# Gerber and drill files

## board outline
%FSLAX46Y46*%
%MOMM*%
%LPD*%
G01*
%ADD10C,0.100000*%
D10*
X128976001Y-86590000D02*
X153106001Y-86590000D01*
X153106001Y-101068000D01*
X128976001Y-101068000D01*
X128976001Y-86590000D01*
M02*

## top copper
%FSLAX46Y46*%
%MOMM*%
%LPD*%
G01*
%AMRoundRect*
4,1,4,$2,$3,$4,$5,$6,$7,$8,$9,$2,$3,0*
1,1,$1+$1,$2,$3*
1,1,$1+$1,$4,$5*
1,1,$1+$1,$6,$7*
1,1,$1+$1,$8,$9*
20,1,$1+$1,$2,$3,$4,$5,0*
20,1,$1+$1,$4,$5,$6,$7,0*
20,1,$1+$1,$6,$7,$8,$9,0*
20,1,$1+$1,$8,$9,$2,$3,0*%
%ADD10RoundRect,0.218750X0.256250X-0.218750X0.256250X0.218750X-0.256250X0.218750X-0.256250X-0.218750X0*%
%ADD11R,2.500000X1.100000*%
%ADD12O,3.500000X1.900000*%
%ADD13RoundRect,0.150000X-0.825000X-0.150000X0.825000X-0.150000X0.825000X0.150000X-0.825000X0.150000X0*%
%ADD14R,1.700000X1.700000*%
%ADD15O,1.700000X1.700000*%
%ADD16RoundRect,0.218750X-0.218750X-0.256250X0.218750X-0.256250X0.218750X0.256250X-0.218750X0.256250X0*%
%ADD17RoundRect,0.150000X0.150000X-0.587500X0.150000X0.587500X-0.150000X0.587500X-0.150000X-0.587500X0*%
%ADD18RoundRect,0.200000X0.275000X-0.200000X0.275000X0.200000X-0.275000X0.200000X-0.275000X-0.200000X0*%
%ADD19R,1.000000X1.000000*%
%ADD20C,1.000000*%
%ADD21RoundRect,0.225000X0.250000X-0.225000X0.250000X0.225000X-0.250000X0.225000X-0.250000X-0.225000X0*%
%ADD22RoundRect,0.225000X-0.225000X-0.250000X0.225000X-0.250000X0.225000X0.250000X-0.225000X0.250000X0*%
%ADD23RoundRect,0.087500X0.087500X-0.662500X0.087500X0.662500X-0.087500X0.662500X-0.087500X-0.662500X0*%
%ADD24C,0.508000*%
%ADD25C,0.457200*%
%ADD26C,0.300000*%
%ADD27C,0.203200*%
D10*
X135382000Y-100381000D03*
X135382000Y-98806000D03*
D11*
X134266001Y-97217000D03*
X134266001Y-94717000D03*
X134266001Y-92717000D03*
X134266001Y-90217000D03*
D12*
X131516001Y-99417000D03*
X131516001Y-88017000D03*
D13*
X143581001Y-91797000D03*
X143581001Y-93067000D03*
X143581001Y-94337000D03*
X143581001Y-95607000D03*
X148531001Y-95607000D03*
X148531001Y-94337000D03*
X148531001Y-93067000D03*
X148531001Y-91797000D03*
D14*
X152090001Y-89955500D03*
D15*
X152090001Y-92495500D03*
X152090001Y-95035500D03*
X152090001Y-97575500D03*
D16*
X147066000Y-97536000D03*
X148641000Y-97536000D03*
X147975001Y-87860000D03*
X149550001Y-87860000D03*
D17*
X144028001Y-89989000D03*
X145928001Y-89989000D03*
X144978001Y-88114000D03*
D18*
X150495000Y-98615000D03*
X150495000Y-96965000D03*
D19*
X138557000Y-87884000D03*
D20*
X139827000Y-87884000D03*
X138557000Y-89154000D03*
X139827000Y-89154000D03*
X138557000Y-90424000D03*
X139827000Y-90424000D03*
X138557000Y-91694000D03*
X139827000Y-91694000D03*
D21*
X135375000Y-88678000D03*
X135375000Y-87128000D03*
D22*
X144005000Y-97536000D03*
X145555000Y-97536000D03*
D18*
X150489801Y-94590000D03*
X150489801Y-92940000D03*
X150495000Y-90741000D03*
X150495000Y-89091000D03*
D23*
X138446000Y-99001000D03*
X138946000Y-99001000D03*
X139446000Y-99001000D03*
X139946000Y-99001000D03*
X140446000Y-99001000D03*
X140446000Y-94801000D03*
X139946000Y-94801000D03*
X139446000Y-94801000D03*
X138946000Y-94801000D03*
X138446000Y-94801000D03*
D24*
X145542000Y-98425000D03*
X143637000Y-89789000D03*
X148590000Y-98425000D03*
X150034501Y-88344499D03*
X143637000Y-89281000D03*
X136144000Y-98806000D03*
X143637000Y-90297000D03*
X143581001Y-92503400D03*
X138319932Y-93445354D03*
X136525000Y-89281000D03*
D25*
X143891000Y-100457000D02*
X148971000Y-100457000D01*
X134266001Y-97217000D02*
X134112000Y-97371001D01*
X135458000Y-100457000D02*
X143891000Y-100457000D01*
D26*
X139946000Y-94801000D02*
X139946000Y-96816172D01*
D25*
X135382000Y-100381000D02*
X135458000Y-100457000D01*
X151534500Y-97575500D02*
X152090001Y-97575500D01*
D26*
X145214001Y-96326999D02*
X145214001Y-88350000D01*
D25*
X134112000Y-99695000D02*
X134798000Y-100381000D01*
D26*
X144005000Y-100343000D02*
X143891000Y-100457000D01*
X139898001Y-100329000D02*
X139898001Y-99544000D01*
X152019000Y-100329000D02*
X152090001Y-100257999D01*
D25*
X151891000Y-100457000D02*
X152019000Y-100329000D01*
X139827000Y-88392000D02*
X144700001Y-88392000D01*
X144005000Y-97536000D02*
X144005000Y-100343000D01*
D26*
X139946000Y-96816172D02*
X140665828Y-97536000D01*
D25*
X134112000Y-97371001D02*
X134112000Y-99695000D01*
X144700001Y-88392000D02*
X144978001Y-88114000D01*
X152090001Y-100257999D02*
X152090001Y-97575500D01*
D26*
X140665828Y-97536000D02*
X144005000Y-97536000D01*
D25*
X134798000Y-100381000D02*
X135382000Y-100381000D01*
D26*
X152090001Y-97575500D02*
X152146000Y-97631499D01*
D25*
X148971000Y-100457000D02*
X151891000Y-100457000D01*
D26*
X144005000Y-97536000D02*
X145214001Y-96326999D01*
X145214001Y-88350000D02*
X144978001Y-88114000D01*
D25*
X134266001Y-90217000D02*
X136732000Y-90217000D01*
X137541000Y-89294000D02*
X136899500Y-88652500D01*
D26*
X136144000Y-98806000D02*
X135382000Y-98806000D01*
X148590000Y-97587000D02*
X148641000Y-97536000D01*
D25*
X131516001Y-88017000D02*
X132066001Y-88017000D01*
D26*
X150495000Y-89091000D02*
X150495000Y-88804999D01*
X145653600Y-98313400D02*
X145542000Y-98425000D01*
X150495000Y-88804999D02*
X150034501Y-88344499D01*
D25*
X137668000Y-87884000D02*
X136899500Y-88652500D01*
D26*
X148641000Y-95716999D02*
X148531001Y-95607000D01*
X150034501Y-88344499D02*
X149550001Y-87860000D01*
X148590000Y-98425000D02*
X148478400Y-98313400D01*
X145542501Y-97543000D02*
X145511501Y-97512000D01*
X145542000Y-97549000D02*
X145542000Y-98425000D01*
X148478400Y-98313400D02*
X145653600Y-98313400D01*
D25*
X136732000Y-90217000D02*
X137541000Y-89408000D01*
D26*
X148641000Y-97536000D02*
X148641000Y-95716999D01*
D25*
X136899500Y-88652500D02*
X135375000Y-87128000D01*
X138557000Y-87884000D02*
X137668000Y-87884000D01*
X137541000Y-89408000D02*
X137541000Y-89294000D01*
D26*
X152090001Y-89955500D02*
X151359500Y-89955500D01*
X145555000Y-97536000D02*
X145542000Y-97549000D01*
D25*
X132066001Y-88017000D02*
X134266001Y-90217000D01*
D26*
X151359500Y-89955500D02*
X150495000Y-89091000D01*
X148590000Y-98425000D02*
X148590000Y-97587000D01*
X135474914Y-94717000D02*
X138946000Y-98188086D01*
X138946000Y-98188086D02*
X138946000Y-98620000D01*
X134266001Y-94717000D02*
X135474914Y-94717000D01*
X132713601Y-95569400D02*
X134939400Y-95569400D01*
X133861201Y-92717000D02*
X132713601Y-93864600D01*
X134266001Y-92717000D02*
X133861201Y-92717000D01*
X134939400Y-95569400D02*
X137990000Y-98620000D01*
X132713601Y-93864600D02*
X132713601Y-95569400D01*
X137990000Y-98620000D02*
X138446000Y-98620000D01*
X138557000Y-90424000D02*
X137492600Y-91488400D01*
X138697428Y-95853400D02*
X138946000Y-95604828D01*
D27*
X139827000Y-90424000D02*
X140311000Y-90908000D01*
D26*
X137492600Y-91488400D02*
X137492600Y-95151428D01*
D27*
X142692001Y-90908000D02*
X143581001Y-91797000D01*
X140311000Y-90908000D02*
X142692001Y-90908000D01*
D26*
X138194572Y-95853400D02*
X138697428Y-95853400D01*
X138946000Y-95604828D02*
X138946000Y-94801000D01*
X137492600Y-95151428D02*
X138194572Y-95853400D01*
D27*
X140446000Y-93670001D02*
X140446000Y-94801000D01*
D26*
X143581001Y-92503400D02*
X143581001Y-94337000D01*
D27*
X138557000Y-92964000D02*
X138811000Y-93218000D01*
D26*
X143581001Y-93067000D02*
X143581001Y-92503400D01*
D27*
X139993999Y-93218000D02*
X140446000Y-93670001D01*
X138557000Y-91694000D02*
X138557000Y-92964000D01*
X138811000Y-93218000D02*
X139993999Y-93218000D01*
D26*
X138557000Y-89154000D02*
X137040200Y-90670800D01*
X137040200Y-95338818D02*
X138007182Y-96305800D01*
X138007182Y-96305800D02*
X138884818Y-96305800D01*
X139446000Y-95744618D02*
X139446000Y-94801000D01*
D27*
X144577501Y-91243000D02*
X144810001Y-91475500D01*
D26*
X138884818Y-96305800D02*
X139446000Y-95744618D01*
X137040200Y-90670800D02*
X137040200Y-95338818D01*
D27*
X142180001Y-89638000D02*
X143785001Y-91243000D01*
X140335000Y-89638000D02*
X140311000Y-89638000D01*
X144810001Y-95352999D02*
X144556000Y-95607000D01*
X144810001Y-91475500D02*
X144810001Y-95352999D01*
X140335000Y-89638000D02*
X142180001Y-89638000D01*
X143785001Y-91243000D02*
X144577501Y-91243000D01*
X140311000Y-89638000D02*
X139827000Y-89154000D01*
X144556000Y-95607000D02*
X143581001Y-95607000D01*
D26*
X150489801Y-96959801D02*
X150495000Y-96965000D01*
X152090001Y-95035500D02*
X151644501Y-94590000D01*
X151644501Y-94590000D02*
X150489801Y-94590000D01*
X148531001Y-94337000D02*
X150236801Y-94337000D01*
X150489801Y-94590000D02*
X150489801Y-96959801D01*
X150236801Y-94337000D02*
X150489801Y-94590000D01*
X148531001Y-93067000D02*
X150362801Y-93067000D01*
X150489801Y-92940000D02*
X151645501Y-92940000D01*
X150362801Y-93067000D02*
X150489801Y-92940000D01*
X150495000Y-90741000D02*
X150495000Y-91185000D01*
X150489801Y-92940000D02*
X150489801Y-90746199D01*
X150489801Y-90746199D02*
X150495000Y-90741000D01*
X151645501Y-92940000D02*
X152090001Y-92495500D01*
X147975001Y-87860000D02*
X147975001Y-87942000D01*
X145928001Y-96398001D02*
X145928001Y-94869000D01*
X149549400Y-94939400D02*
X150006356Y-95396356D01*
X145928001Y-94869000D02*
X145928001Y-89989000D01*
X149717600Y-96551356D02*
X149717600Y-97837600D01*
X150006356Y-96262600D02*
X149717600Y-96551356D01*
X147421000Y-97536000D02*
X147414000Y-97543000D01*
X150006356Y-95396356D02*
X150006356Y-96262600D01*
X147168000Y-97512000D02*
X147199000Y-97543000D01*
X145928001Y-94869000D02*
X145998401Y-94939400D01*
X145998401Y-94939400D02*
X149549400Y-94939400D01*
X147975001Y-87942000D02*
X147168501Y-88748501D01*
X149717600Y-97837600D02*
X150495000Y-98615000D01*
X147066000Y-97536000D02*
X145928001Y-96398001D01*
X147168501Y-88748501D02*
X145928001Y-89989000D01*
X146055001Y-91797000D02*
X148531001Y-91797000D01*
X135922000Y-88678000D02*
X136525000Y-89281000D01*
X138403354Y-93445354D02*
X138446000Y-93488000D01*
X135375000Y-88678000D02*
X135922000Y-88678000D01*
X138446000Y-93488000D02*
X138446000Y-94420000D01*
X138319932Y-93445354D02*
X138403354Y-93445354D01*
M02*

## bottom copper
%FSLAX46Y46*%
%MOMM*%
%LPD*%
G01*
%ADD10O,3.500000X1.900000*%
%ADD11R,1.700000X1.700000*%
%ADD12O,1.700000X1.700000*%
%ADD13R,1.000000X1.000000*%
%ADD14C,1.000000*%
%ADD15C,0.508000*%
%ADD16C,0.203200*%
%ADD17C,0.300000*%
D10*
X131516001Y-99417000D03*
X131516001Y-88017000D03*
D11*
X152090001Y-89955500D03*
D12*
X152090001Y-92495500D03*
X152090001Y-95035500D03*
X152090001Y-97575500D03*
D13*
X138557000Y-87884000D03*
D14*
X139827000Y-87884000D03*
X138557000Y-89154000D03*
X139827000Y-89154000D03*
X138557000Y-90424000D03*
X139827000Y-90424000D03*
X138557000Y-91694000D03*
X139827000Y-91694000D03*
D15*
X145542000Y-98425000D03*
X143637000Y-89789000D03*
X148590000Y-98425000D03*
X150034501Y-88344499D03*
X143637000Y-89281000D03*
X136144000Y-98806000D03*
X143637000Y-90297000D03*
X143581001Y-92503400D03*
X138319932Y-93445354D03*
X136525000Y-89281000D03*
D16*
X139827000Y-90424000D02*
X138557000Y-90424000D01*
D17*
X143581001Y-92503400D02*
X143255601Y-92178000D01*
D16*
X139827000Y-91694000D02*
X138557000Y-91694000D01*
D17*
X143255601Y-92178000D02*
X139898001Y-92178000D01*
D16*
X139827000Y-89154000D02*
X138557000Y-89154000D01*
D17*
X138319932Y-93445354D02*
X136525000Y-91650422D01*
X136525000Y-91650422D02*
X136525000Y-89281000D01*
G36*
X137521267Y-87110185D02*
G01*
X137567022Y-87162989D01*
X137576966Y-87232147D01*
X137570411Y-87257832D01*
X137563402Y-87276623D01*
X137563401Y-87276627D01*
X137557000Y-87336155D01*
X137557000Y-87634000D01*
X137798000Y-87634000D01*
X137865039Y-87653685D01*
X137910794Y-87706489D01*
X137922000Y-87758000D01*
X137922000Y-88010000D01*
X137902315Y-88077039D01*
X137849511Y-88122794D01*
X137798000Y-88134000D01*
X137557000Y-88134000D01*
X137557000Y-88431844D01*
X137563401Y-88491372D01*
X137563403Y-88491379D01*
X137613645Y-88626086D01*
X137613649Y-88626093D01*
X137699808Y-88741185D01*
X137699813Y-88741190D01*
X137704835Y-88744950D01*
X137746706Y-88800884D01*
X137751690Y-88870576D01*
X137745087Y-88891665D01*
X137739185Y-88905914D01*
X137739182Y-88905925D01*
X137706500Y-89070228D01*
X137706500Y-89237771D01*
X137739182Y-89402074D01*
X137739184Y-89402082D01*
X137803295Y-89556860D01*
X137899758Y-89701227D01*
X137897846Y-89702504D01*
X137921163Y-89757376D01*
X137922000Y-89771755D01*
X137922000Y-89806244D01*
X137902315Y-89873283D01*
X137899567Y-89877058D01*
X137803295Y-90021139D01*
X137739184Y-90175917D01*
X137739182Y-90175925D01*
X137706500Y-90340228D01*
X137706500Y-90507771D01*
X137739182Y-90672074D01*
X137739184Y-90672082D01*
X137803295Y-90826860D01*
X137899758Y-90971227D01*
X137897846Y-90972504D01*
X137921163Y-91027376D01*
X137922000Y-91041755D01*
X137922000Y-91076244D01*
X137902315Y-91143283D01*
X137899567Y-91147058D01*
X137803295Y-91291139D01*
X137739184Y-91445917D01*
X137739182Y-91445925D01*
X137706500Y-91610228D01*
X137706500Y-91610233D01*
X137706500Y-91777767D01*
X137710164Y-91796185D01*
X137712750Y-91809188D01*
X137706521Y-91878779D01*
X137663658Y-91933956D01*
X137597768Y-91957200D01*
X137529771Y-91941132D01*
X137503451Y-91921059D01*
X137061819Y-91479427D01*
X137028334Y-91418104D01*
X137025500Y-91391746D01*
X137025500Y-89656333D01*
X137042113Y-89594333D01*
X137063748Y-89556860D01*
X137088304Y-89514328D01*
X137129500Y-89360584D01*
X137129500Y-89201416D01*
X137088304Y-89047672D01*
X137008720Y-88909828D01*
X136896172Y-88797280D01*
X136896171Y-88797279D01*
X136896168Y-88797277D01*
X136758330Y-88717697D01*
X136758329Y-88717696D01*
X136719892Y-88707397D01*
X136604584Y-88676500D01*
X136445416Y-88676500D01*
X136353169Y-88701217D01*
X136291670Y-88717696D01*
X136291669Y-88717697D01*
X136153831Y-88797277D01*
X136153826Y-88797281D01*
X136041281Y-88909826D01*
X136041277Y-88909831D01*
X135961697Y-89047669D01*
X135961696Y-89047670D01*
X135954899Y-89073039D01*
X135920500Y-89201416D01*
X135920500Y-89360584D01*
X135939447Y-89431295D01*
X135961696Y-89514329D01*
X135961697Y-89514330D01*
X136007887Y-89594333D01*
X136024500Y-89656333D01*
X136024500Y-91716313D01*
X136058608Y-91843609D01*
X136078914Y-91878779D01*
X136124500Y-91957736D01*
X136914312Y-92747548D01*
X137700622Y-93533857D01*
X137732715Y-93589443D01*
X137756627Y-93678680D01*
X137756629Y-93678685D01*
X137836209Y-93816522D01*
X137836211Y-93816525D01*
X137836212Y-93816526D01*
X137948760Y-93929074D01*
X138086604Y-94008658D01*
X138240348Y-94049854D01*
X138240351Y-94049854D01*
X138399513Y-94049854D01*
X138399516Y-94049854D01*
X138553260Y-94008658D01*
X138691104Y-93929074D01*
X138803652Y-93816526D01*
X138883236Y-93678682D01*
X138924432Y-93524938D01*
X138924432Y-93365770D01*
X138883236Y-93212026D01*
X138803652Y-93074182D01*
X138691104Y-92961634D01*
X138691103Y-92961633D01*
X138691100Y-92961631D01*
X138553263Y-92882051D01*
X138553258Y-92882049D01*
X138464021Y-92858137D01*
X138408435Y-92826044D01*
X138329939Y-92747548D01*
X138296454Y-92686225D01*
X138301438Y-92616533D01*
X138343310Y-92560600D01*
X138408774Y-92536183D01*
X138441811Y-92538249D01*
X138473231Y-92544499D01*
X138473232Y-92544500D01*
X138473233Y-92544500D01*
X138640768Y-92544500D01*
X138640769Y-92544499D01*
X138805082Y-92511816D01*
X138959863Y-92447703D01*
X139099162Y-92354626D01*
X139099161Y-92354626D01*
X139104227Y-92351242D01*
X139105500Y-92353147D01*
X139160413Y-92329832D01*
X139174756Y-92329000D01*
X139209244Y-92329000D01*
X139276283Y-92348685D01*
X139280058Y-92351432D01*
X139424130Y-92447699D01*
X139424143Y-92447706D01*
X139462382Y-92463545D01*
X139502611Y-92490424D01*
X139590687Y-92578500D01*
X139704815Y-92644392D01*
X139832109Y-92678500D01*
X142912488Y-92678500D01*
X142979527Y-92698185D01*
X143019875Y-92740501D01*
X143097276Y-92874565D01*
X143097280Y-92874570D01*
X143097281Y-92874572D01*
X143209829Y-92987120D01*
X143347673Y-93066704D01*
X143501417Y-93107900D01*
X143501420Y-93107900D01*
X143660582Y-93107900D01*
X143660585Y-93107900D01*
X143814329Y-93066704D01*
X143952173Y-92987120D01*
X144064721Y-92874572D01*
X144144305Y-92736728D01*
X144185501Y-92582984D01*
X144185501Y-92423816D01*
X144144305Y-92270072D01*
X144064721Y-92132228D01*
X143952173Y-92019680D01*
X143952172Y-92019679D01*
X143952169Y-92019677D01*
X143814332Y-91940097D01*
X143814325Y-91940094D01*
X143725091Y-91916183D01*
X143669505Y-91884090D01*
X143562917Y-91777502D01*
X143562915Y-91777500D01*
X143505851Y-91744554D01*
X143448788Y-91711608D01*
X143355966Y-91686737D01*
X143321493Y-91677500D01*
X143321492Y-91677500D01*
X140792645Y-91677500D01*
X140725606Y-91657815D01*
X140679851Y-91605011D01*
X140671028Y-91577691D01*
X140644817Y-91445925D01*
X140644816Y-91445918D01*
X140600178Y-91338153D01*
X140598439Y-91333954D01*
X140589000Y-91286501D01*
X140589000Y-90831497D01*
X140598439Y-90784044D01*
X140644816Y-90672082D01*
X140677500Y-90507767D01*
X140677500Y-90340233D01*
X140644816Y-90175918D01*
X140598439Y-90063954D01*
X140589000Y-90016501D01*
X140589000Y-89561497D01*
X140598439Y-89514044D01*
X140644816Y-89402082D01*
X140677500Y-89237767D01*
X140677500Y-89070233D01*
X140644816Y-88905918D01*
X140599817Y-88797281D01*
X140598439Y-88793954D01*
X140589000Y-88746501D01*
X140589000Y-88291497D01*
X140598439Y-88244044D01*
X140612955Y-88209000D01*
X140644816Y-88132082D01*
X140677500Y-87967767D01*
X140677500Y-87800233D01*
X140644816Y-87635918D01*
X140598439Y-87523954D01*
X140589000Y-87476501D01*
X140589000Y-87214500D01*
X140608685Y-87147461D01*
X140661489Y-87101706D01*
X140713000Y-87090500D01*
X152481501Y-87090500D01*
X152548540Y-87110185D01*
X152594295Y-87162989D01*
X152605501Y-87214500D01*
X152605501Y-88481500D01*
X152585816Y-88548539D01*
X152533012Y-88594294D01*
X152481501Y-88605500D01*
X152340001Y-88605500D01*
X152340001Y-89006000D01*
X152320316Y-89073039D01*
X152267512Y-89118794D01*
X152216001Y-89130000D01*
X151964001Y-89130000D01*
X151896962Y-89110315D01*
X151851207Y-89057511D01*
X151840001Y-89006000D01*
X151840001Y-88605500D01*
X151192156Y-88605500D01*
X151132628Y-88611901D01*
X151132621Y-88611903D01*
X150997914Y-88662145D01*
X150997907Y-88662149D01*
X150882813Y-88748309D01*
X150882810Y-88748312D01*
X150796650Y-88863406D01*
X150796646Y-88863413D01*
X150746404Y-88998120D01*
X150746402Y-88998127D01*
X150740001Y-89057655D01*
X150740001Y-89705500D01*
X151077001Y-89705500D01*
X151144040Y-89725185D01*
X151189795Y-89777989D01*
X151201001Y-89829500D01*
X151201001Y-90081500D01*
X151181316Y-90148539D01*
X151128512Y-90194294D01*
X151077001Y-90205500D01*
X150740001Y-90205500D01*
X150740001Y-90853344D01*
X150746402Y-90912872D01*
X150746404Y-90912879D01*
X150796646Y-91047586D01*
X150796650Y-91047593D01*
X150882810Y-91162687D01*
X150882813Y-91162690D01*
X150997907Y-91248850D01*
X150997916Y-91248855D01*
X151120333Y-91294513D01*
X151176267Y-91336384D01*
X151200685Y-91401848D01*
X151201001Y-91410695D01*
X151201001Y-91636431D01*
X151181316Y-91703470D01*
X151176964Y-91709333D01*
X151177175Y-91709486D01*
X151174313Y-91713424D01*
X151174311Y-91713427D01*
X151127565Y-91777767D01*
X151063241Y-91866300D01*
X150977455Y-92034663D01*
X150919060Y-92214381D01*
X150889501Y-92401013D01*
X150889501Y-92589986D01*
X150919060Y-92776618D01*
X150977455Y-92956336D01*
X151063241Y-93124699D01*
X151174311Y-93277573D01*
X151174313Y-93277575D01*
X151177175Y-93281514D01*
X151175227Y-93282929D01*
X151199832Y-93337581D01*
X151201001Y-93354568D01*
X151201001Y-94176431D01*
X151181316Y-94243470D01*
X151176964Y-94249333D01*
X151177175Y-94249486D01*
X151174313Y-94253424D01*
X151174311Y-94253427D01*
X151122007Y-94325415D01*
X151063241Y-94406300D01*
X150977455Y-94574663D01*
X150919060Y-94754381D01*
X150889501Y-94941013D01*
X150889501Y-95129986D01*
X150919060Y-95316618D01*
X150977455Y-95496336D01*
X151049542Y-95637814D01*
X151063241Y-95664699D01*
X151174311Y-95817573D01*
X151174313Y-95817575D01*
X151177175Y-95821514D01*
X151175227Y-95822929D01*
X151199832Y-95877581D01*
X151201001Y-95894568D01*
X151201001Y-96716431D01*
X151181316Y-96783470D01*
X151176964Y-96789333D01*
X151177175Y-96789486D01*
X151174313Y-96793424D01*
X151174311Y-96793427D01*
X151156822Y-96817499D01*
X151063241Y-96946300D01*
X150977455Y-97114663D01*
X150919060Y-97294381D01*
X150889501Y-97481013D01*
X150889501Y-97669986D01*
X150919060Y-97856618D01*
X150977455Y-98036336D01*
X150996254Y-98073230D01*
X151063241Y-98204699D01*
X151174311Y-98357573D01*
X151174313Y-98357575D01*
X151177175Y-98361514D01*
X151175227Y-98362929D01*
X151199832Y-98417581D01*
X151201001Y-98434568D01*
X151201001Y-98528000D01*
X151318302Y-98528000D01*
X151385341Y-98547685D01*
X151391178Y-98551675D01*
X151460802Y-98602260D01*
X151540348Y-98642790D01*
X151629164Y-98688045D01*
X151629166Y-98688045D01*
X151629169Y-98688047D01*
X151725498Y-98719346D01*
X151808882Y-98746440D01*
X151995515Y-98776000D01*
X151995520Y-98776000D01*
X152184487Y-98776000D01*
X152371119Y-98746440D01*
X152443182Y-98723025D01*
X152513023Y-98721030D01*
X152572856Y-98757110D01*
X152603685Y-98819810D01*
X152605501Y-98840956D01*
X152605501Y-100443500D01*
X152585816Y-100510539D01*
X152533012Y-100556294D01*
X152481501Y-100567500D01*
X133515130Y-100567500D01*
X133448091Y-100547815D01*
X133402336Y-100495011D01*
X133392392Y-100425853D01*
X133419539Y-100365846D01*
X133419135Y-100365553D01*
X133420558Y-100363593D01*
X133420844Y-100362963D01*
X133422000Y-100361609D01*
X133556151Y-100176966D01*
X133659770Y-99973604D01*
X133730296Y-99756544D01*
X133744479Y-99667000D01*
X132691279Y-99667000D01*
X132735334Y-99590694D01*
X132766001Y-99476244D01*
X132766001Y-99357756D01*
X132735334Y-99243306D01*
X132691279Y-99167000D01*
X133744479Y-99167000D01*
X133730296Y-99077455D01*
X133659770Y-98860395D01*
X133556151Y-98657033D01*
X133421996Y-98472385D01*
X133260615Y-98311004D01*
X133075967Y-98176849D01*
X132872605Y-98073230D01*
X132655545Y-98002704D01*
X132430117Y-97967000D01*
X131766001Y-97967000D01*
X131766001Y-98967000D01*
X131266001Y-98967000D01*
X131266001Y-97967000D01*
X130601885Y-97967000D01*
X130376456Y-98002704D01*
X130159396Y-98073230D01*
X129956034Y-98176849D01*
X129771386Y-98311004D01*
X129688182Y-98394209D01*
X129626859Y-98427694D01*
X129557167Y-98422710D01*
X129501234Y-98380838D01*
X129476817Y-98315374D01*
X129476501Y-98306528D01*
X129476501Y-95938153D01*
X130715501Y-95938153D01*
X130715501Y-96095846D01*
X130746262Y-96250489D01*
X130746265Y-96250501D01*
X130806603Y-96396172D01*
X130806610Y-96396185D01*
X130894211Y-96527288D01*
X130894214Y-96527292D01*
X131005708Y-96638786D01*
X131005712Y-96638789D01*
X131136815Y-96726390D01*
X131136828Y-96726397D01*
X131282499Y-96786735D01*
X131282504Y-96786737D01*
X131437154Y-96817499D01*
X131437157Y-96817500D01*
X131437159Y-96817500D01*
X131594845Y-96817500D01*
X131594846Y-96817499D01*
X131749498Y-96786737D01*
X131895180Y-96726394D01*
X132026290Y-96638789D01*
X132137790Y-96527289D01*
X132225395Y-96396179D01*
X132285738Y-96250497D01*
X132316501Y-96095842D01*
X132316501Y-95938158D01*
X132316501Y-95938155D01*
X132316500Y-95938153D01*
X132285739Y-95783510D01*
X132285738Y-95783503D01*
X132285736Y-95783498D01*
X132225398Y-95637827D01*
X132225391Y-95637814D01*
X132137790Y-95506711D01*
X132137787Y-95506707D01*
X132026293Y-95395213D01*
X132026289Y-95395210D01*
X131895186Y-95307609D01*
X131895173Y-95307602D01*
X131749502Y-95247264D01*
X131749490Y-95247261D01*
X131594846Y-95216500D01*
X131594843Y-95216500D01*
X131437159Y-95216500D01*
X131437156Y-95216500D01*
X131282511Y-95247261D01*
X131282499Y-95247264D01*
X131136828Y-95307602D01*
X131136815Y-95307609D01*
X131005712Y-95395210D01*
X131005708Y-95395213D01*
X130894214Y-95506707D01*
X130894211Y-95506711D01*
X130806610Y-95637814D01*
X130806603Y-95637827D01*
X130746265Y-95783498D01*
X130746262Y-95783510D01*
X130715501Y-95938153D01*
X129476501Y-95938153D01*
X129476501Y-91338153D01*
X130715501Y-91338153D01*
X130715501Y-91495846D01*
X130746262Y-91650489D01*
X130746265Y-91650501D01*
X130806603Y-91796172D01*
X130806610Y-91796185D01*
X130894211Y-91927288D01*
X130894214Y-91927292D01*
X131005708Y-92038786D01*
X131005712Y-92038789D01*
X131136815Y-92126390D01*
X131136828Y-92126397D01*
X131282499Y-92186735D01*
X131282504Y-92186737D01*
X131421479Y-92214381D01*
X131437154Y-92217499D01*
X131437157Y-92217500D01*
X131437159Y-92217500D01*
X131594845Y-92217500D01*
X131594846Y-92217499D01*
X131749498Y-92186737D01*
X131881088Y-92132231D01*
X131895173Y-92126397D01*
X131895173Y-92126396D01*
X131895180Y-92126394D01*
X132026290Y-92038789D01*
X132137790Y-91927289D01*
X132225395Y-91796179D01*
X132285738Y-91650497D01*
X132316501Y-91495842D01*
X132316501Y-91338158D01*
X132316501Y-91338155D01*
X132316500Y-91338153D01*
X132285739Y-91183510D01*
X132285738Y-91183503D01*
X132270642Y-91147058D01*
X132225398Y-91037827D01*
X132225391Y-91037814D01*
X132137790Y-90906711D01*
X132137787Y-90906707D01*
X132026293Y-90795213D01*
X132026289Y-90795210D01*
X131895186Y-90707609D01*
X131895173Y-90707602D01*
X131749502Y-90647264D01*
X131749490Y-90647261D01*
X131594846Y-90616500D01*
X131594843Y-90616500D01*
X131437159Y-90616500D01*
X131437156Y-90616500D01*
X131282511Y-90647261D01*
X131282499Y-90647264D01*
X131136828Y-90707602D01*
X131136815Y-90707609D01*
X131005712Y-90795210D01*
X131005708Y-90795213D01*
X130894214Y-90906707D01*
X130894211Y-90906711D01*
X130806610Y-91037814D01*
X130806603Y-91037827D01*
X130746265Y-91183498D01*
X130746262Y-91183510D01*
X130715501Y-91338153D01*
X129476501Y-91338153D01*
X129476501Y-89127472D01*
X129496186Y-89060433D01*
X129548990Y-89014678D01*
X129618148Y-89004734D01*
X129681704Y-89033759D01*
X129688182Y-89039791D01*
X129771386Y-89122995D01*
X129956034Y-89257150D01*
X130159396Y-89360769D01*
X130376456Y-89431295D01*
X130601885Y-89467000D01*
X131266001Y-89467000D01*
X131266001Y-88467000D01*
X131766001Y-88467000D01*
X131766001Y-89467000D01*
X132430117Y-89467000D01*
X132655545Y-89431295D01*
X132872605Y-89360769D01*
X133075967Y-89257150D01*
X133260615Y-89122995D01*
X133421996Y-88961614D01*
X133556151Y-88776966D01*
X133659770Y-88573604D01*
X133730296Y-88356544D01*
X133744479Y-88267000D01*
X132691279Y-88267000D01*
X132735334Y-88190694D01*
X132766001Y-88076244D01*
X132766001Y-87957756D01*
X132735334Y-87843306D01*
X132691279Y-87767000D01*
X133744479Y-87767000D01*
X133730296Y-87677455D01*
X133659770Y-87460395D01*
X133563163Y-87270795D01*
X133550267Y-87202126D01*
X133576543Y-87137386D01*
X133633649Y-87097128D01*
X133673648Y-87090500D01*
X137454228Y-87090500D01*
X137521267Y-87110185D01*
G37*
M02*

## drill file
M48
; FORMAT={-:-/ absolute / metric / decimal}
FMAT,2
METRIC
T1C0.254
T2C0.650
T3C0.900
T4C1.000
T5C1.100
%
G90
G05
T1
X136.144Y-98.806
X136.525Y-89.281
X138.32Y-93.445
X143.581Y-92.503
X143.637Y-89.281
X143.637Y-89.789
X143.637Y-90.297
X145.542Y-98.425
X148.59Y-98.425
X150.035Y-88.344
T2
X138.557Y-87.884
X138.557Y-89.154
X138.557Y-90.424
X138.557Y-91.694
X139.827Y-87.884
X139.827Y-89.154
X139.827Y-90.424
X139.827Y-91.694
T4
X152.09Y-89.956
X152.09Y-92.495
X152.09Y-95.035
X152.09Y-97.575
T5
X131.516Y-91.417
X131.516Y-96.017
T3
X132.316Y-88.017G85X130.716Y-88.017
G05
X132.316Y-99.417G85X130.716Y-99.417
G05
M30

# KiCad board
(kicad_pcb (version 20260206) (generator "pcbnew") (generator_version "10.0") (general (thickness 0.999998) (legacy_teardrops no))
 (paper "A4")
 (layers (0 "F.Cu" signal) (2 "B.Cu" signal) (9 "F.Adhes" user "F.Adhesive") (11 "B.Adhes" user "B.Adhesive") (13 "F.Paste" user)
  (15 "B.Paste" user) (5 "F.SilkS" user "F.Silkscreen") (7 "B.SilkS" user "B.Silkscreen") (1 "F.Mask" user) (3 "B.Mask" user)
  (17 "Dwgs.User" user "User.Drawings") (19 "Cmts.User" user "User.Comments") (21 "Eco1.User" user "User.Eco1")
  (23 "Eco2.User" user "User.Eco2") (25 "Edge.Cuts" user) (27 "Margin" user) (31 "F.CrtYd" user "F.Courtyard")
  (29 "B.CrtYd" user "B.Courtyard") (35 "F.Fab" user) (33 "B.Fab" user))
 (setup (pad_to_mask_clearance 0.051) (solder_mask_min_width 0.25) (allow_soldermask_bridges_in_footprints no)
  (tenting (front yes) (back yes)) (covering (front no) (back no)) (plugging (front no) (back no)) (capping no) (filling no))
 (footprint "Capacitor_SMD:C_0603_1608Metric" (layer "F.Cu") (at 135.382 99.5935 90)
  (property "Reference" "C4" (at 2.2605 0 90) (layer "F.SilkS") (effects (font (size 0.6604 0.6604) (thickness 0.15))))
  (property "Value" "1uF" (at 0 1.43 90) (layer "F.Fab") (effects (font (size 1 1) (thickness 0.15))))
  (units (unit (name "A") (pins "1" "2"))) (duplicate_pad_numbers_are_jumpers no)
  (pad "1" smd roundrect (at -0.7875 0 90) (size 0.875 0.95) (layers "F.Cu" "F.Mask" "F.Paste") (roundrect_rratio 0.25) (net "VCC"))
  (pad "2" smd roundrect (at 0.7875 0 90) (size 0.875 0.95) (layers "F.Cu" "F.Mask" "F.Paste") (roundrect_rratio 0.25) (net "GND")))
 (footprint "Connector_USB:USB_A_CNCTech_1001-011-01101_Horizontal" (layer "F.Cu") (at 124.616001 93.717 180)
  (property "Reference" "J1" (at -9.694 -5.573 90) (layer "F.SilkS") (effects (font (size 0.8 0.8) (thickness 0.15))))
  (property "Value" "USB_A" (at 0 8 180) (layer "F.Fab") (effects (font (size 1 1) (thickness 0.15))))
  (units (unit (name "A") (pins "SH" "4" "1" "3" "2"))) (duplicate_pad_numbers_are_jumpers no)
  (pad "" np_thru_hole circle (at -6.9 -2.3 180) (size 1.1 1.1) (drill 1.1) (layers "*.Cu" "*.Mask"))
  (pad "" np_thru_hole circle (at -6.9 2.3 180) (size 1.1 1.1) (drill 1.1) (layers "*.Cu" "*.Mask"))
  (pad "1" smd rect (at -9.65 -3.5 180) (size 2.5 1.1) (layers "F.Cu" "F.Mask" "F.Paste") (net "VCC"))
  (pad "2" smd rect (at -9.65 -1 180) (size 2.5 1.1) (layers "F.Cu" "F.Mask" "F.Paste") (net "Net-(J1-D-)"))
  (pad "3" smd rect (at -9.65 1 180) (size 2.5 1.1) (layers "F.Cu" "F.Mask" "F.Paste") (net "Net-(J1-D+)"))
  (pad "4" smd rect (at -9.65 3.5 180) (size 2.5 1.1) (layers "F.Cu" "F.Mask" "F.Paste") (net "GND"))
  (pad "SH" thru_hole oval (at -6.9 -5.7 180) (size 3.5 1.9) (drill oval 2.5 0.9) (layers "*.Cu" "*.Mask") (remove_unused_layers no)
   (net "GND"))
  (pad "SH" thru_hole oval (at -6.9 5.7 180) (size 3.5 1.9) (drill oval 2.5 0.9) (layers "*.Cu" "*.Mask") (remove_unused_layers no)
   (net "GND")))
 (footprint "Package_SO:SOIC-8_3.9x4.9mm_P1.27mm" (layer "F.Cu") (at 146.056001 93.702)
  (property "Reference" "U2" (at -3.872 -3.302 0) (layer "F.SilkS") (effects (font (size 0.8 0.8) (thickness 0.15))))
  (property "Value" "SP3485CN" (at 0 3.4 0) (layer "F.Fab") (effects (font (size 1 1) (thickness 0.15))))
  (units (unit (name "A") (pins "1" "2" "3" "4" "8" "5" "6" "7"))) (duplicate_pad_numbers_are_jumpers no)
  (pad "1" smd roundrect (at -2.475 -1.905) (size 1.95 0.6) (layers "F.Cu" "F.Mask" "F.Paste") (roundrect_rratio 0.25) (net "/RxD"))
  (pad "2" smd roundrect (at -2.475 -0.635) (size 1.95 0.6) (layers "F.Cu" "F.Mask" "F.Paste") (roundrect_rratio 0.25) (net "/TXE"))
  (pad "3" smd roundrect (at -2.475 0.635) (size 1.95 0.6) (layers "F.Cu" "F.Mask" "F.Paste") (roundrect_rratio 0.25) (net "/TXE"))
  (pad "4" smd roundrect (at -2.475 1.905) (size 1.95 0.6) (layers "F.Cu" "F.Mask" "F.Paste") (roundrect_rratio 0.25) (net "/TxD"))
  (pad "5" smd roundrect (at 2.475 1.905) (size 1.95 0.6) (layers "F.Cu" "F.Mask" "F.Paste") (roundrect_rratio 0.25) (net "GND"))
  (pad "6" smd roundrect (at 2.475 0.635) (size 1.95 0.6) (layers "F.Cu" "F.Mask" "F.Paste") (roundrect_rratio 0.25) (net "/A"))
  (pad "7" smd roundrect (at 2.475 -0.635) (size 1.95 0.6) (layers "F.Cu" "F.Mask" "F.Paste") (roundrect_rratio 0.25) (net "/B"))
  (pad "8" smd roundrect (at 2.475 -1.905) (size 1.95 0.6) (layers "F.Cu" "F.Mask" "F.Paste") (roundrect_rratio 0.25) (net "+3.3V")))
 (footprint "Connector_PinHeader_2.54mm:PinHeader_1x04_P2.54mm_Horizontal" (layer "F.Cu") (at 152.090001 89.9555)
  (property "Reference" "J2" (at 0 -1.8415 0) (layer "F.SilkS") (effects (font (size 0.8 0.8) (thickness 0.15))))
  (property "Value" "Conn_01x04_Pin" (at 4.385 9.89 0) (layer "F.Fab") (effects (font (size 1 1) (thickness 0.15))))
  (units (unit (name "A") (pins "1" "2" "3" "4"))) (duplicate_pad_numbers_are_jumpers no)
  (pad "1" thru_hole rect (at 0 0) (size 1.7 1.7) (drill 1) (layers "*.Cu" "*.Mask") (remove_unused_layers no) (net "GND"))
  (pad "2" thru_hole oval (at 0 2.54) (size 1.7 1.7) (drill 1) (layers "*.Cu" "*.Mask") (remove_unused_layers no) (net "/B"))
  (pad "3" thru_hole oval (at 0 5.08) (size 1.7 1.7) (drill 1) (layers "*.Cu" "*.Mask") (remove_unused_layers no) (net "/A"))
  (pad "4" thru_hole oval (at 0 7.62) (size 1.7 1.7) (drill 1) (layers "*.Cu" "*.Mask") (remove_unused_layers no) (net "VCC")))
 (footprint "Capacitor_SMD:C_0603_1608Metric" (layer "F.Cu") (at 147.8535 97.536)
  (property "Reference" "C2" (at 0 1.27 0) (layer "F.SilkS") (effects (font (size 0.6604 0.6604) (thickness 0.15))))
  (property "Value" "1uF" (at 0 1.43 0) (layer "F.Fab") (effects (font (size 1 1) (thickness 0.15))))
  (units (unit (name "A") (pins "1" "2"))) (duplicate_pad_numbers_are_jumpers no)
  (pad "1" smd roundrect (at -0.7875 0) (size 0.875 0.95) (layers "F.Cu" "F.Mask" "F.Paste") (roundrect_rratio 0.25) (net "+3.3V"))
  (pad "2" smd roundrect (at 0.7875 0) (size 0.875 0.95) (layers "F.Cu" "F.Mask" "F.Paste") (roundrect_rratio 0.25) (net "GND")))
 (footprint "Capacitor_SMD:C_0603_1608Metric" (layer "F.Cu") (at 148.762501 87.86)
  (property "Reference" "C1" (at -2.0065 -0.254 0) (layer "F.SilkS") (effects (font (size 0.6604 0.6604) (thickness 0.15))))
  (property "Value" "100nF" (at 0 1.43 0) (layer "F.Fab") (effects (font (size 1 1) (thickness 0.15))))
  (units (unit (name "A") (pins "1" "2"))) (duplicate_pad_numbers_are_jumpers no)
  (pad "1" smd roundrect (at -0.7875 0) (size 0.875 0.95) (layers "F.Cu" "F.Mask" "F.Paste") (roundrect_rratio 0.25) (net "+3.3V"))
  (pad "2" smd roundrect (at 0.7875 0) (size 0.875 0.95) (layers "F.Cu" "F.Mask" "F.Paste") (roundrect_rratio 0.25) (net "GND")))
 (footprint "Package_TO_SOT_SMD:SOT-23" (layer "F.Cu") (at 144.978001 89.0515 90)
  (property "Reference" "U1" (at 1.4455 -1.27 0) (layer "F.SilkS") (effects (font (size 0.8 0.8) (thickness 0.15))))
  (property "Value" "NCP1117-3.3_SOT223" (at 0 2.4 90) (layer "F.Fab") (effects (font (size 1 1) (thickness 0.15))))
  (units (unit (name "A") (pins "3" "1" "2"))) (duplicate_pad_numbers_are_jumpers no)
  (pad "1" smd roundrect (at -0.9375 -0.95 90) (size 1.475 0.6) (layers "F.Cu" "F.Mask" "F.Paste") (roundrect_rratio 0.25) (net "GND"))
  (pad "2" smd roundrect (at -0.9375 0.95 90) (size 1.475 0.6) (layers "F.Cu" "F.Mask" "F.Paste") (roundrect_rratio 0.25) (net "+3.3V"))
  (pad "3" smd roundrect (at 0.9375 0 90) (size 1.475 0.6) (layers "F.Cu" "F.Mask" "F.Paste") (roundrect_rratio 0.25) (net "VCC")))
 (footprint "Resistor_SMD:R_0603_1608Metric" (layer "F.Cu") (at 150.495 97.79 90)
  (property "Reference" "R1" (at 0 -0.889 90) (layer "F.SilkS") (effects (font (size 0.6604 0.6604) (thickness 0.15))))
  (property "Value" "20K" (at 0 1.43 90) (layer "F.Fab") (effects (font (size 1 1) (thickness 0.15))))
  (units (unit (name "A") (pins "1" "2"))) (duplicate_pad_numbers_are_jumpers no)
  (pad "1" smd roundrect (at -0.825 0 90) (size 0.8 0.95) (layers "F.Cu" "F.Mask" "F.Paste") (roundrect_rratio 0.25) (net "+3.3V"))
  (pad "2" smd roundrect (at 0.825 0 90) (size 0.8 0.95) (layers "F.Cu" "F.Mask" "F.Paste") (roundrect_rratio 0.25) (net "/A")))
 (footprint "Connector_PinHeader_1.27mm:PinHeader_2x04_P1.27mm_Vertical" (layer "F.Cu") (at 138.557 87.884)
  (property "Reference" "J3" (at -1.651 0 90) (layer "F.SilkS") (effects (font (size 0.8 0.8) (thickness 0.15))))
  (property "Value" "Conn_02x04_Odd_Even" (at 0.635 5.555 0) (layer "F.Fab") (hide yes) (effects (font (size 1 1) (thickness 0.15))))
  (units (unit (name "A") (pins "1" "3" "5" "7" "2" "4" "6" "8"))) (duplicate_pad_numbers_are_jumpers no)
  (pad "1" thru_hole rect (at 0 0) (size 1 1) (drill 0.65) (layers "*.Cu" "*.Mask") (remove_unused_layers no) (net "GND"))
  (pad "2" thru_hole circle (at 1.27 0) (size 1 1) (drill 0.65) (layers "*.Cu" "*.Mask") (remove_unused_layers no) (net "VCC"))
  (pad "3" thru_hole circle (at 0 1.27) (size 1 1) (drill 0.65) (layers "*.Cu" "*.Mask") (remove_unused_layers no) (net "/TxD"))
  (pad "4" thru_hole circle (at 1.27 1.27) (size 1 1) (drill 0.65) (layers "*.Cu" "*.Mask") (remove_unused_layers no) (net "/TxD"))
  (pad "5" thru_hole circle (at 0 2.54) (size 1 1) (drill 0.65) (layers "*.Cu" "*.Mask") (remove_unused_layers no) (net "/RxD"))
  (pad "6" thru_hole circle (at 1.27 2.54) (size 1 1) (drill 0.65) (layers "*.Cu" "*.Mask") (remove_unused_layers no) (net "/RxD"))
  (pad "7" thru_hole circle (at 0 3.81) (size 1 1) (drill 0.65) (layers "*.Cu" "*.Mask") (remove_unused_layers no) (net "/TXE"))
  (pad "8" thru_hole circle (at 1.27 3.81) (size 1 1) (drill 0.65) (layers "*.Cu" "*.Mask") (remove_unused_layers no) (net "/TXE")))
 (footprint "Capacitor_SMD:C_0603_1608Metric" (layer "F.Cu") (at 135.375 87.903 90)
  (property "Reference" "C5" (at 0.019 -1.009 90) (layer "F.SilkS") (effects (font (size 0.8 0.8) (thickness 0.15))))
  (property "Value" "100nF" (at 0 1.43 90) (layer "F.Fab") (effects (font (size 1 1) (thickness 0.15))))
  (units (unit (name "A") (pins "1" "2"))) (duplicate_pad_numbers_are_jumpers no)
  (pad "1" smd roundrect (at -0.775 0 90) (size 0.9 0.95) (layers "F.Cu" "F.Mask" "F.Paste") (roundrect_rratio 0.25) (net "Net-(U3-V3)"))
  (pad "2" smd roundrect (at 0.775 0 90) (size 0.9 0.95) (layers "F.Cu" "F.Mask" "F.Paste") (roundrect_rratio 0.25) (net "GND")))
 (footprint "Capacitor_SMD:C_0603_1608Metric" (layer "F.Cu") (at 144.78 97.536)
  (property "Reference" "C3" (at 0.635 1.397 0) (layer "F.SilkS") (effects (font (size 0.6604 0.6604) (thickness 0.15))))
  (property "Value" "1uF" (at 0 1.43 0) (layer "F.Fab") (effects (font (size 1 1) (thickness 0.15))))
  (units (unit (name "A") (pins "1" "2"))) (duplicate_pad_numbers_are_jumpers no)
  (pad "1" smd roundrect (at -0.775 0) (size 0.9 0.95) (layers "F.Cu" "F.Mask" "F.Paste") (roundrect_rratio 0.25) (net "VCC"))
  (pad "2" smd roundrect (at 0.775 0) (size 0.9 0.95) (layers "F.Cu" "F.Mask" "F.Paste") (roundrect_rratio 0.25) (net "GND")))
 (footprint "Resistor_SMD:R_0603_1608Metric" (layer "F.Cu") (at 150.489801 93.765 90)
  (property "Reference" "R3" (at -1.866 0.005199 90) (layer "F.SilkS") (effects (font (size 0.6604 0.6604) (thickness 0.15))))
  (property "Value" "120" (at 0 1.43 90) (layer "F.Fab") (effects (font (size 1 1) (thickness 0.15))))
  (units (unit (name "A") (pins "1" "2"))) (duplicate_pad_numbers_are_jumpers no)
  (pad "1" smd roundrect (at -0.825 0 90) (size 0.8 0.95) (layers "F.Cu" "F.Mask" "F.Paste") (roundrect_rratio 0.25) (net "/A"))
  (pad "2" smd roundrect (at 0.825 0 90) (size 0.8 0.95) (layers "F.Cu" "F.Mask" "F.Paste") (roundrect_rratio 0.25) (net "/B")))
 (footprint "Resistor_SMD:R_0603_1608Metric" (layer "F.Cu") (at 150.495 89.916 90)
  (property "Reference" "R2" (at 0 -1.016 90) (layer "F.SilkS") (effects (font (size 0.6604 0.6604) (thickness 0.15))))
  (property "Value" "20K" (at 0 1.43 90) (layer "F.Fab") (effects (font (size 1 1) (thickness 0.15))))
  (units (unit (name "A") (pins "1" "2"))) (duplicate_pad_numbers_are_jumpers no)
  (pad "1" smd roundrect (at -0.825 0 90) (size 0.8 0.95) (layers "F.Cu" "F.Mask" "F.Paste") (roundrect_rratio 0.25) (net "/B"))
  (pad "2" smd roundrect (at 0.825 0 90) (size 0.8 0.95) (layers "F.Cu" "F.Mask" "F.Paste") (roundrect_rratio 0.25) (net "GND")))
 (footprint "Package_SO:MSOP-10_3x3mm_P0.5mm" (layer "F.Cu") (at 139.446 96.901 90)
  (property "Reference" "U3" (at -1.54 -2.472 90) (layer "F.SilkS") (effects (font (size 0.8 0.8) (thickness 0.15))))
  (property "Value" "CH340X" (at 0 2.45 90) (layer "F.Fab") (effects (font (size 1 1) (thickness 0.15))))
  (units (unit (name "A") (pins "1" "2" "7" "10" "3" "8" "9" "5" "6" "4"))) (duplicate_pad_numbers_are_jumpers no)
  (pad "1" smd roundrect (at -2.1 -1 90) (size 1.5 0.35) (layers "F.Cu" "F.Mask" "F.Paste") (roundrect_rratio 0.25) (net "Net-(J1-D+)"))
  (pad "2" smd roundrect (at -2.1 -0.5 90) (size 1.5 0.35) (layers "F.Cu" "F.Mask" "F.Paste") (roundrect_rratio 0.25) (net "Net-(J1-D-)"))
  (pad "3" smd roundrect (at -2.1 0 90) (size 1.5 0.35) (layers "F.Cu" "F.Mask" "F.Paste") (roundrect_rratio 0.25) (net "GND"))
  (pad "4" smd roundrect (at -2.1 0.5 90) (size 1.5 0.35) (layers "F.Cu" "F.Mask" "F.Paste") (roundrect_rratio 0.25)
   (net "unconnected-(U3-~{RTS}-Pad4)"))
  (pad "5" smd roundrect (at -2.1 1 90) (size 1.5 0.35) (layers "F.Cu" "F.Mask" "F.Paste") (roundrect_rratio 0.25)
   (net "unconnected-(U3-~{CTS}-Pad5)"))
  (pad "6" smd roundrect (at 2.1 1 90) (size 1.5 0.35) (layers "F.Cu" "F.Mask" "F.Paste") (roundrect_rratio 0.25) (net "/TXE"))
  (pad "7" smd roundrect (at 2.1 0.5 90) (size 1.5 0.35) (layers "F.Cu" "F.Mask" "F.Paste") (roundrect_rratio 0.25) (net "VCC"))
  (pad "8" smd roundrect (at 2.1 0 90) (size 1.5 0.35) (layers "F.Cu" "F.Mask" "F.Paste") (roundrect_rratio 0.25) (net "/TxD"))
  (pad "9" smd roundrect (at 2.1 -0.5 90) (size 1.5 0.35) (layers "F.Cu" "F.Mask" "F.Paste") (roundrect_rratio 0.25) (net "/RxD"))
  (pad "10" smd roundrect (at 2.1 -1 90) (size 1.5 0.35) (layers "F.Cu" "F.Mask" "F.Paste") (roundrect_rratio 0.25) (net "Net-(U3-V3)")))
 (gr_rect (start 128.976001 86.59) (end 153.106001 101.068) (stroke (width 0.1) (type solid)) (fill no) (layer "Edge.Cuts"))
 (segment (start 143.891 100.457) (end 148.971 100.457) (width 0.4572) (layer "F.Cu") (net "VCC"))
 (segment (start 134.266001 97.217) (end 134.112 97.371001) (width 0.4572) (layer "F.Cu") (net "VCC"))
 (segment (start 135.458 100.457) (end 143.891 100.457) (width 0.4572) (layer "F.Cu") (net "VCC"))
 (segment (start 139.946 94.801) (end 139.946 96.816172) (width 0.3) (layer "F.Cu") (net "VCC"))
 (segment (start 135.382 100.381) (end 135.458 100.457) (width 0.4572) (layer "F.Cu") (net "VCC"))
 (segment (start 151.5345 97.5755) (end 152.090001 97.5755) (width 0.4572) (layer "F.Cu") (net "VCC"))
 (segment (start 145.214001 96.326999) (end 145.214001 88.35) (width 0.3) (layer "F.Cu") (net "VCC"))
 (segment (start 134.112 99.695) (end 134.798 100.381) (width 0.4572) (layer "F.Cu") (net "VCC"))
 (segment (start 144.005 100.343) (end 143.891 100.457) (width 0.3) (layer "F.Cu") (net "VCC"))
 (segment (start 139.898001 100.329) (end 139.898001 99.544) (width 0.3) (layer "F.Cu") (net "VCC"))
 (segment (start 152.019 100.329) (end 152.090001 100.257999) (width 0.3) (layer "F.Cu") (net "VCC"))
 (segment (start 151.891 100.457) (end 152.019 100.329) (width 0.4572) (layer "F.Cu") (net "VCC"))
 (segment (start 139.827 88.392) (end 144.700001 88.392) (width 0.4572) (layer "F.Cu") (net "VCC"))
 (segment (start 144.005 97.536) (end 144.005 100.343) (width 0.4572) (layer "F.Cu") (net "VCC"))
 (segment (start 139.946 96.816172) (end 140.665828 97.536) (width 0.3) (layer "F.Cu") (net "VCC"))
 (segment (start 134.112 97.371001) (end 134.112 99.695) (width 0.4572) (layer "F.Cu") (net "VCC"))
 (segment (start 144.700001 88.392) (end 144.978001 88.114) (width 0.4572) (layer "F.Cu") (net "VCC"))
 (segment (start 152.090001 100.257999) (end 152.090001 97.5755) (width 0.4572) (layer "F.Cu") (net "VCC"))
 (segment (start 140.665828 97.536) (end 144.005 97.536) (width 0.3) (layer "F.Cu") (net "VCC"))
 (segment (start 134.798 100.381) (end 135.382 100.381) (width 0.4572) (layer "F.Cu") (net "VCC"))
 (segment (start 152.090001 97.5755) (end 152.146 97.631499) (width 0.3) (layer "F.Cu") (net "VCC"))
 (segment (start 148.971 100.457) (end 151.891 100.457) (width 0.4572) (layer "F.Cu") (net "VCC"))
 (segment (start 144.005 97.536) (end 145.214001 96.326999) (width 0.3) (layer "F.Cu") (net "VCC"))
 (segment (start 145.214001 88.35) (end 144.978001 88.114) (width 0.3) (layer "F.Cu") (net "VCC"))
 (segment (start 134.266001 90.217) (end 136.732 90.217) (width 0.4572) (layer "F.Cu") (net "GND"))
 (segment (start 137.541 89.294) (end 136.8995 88.6525) (width 0.4572) (layer "F.Cu") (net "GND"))
 (segment (start 136.144 98.806) (end 135.382 98.806) (width 0.3) (layer "F.Cu") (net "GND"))
 (segment (start 148.59 97.587) (end 148.641 97.536) (width 0.3) (layer "F.Cu") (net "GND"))
 (segment (start 131.516001 88.017) (end 132.066001 88.017) (width 0.4572) (layer "F.Cu") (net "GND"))
 (segment (start 150.495 89.091) (end 150.495 88.804999) (width 0.3) (layer "F.Cu") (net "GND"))
 (segment (start 145.6536 98.3134) (end 145.542 98.425) (width 0.3) (layer "F.Cu") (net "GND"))
 (segment (start 150.495 88.804999) (end 150.034501 88.344499) (width 0.3) (layer "F.Cu") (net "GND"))
 (segment (start 137.668 87.884) (end 136.8995 88.6525) (width 0.4572) (layer "F.Cu") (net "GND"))
 (segment (start 148.641 95.716999) (end 148.531001 95.607) (width 0.3) (layer "F.Cu") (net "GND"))
 (segment (start 150.034501 88.344499) (end 149.550001 87.86) (width 0.3) (layer "F.Cu") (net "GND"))
 (segment (start 148.59 98.425) (end 148.4784 98.3134) (width 0.3) (layer "F.Cu") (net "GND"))
 (segment (start 145.542501 97.543) (end 145.511501 97.512) (width 0.3) (layer "F.Cu") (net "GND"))
 (segment (start 145.542 97.549) (end 145.542 98.425) (width 0.3) (layer "F.Cu") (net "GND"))
 (segment (start 148.4784 98.3134) (end 145.6536 98.3134) (width 0.3) (layer "F.Cu") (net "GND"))
 (segment (start 136.732 90.217) (end 137.541 89.408) (width 0.4572) (layer "F.Cu") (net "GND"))
 (segment (start 148.641 97.536) (end 148.641 95.716999) (width 0.3) (layer "F.Cu") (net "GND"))
 (segment (start 136.8995 88.6525) (end 135.375 87.128) (width 0.4572) (layer "F.Cu") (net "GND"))
 (segment (start 138.557 87.884) (end 137.668 87.884) (width 0.4572) (layer "F.Cu") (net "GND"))
 (segment (start 137.541 89.408) (end 137.541 89.294) (width 0.4572) (layer "F.Cu") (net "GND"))
 (segment (start 152.090001 89.9555) (end 151.3595 89.9555) (width 0.3) (layer "F.Cu") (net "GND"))
 (segment (start 145.555 97.536) (end 145.542 97.549) (width 0.3) (layer "F.Cu") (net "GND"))
 (segment (start 132.066001 88.017) (end 134.266001 90.217) (width 0.4572) (layer "F.Cu") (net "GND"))
 (segment (start 151.3595 89.9555) (end 150.495 89.091) (width 0.3) (layer "F.Cu") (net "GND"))
 (segment (start 148.59 98.425) (end 148.59 97.587) (width 0.3) (layer "F.Cu") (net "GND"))
 (via (at 145.542 98.425) (size 0.508) (drill 0.254) (layers "F.Cu" "B.Cu") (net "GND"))
 (via (at 143.637 89.789) (size 0.508) (drill 0.254) (layers "F.Cu" "B.Cu") (free yes) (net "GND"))
 (via (at 148.59 98.425) (size 0.508) (drill 0.254) (layers "F.Cu" "B.Cu") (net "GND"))
 (via (at 150.034501 88.344499) (size 0.508) (drill 0.254) (layers "F.Cu" "B.Cu") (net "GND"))
 (via (at 143.637 89.281) (size 0.508) (drill 0.254) (layers "F.Cu" "B.Cu") (free yes) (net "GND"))
 (via (at 136.144 98.806) (size 0.508) (drill 0.254) (layers "F.Cu" "B.Cu") (free yes) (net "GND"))
 (via (at 143.637 90.297) (size 0.508) (drill 0.254) (layers "F.Cu" "B.Cu") (free yes) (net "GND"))
 (segment (start 135.474914 94.717) (end 138.946 98.188086) (width 0.3) (layer "F.Cu") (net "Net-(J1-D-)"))
 (segment (start 138.946 98.188086) (end 138.946 98.62) (width 0.3) (layer "F.Cu") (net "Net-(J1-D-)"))
 (segment (start 134.266001 94.717) (end 135.474914 94.717) (width 0.3) (layer "F.Cu") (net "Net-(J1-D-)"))
 (segment (start 132.713601 95.5694) (end 134.9394 95.5694) (width 0.3) (layer "F.Cu") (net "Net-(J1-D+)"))
 (segment (start 133.861201 92.717) (end 132.713601 93.8646) (width 0.3) (layer "F.Cu") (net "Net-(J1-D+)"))
 (segment (start 134.266001 92.717) (end 133.861201 92.717) (width 0.3) (layer "F.Cu") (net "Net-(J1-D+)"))
 (segment (start 134.9394 95.5694) (end 137.99 98.62) (width 0.3) (layer "F.Cu") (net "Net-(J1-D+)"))
 (segment (start 132.713601 93.8646) (end 132.713601 95.5694) (width 0.3) (layer "F.Cu") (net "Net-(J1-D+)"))
 (segment (start 137.99 98.62) (end 138.446 98.62) (width 0.3) (layer "F.Cu") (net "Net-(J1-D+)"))
 (segment (start 138.557 90.424) (end 137.4926 91.4884) (width 0.3) (layer "F.Cu") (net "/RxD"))
 (segment (start 138.697428 95.8534) (end 138.946 95.604828) (width 0.3) (layer "F.Cu") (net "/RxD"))
 (segment (start 139.827 90.424) (end 140.311 90.908) (width 0.2032) (layer "F.Cu") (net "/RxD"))
 (segment (start 137.4926 91.4884) (end 137.4926 95.151428) (width 0.3) (layer "F.Cu") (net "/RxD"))
 (segment (start 142.692001 90.908) (end 143.581001 91.797) (width 0.2032) (layer "F.Cu") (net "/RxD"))
 (segment (start 140.311 90.908) (end 142.692001 90.908) (width 0.2032) (layer "F.Cu") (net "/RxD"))
 (segment (start 138.194572 95.8534) (end 138.697428 95.8534) (width 0.3) (layer "F.Cu") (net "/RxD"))
 (segment (start 138.946 95.604828) (end 138.946 94.801) (width 0.3) (layer "F.Cu") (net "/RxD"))
 (segment (start 137.4926 95.151428) (end 138.194572 95.8534) (width 0.3) (layer "F.Cu") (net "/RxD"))
 (segment (start 139.827 90.424) (end 138.557 90.424) (width 0.2032) (layer "B.Cu") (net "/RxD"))
 (segment (start 140.446 93.670001) (end 140.446 94.801) (width 0.2032) (layer "F.Cu") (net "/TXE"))
 (segment (start 143.581001 92.5034) (end 143.581001 94.337) (width 0.3) (layer "F.Cu") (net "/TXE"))
 (segment (start 138.557 92.964) (end 138.811 93.218) (width 0.2032) (layer "F.Cu") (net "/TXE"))
 (segment (start 143.581001 93.067) (end 143.581001 92.5034) (width 0.3) (layer "F.Cu") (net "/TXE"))
 (segment (start 139.993999 93.218) (end 140.446 93.670001) (width 0.2032) (layer "F.Cu") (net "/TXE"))
 (segment (start 138.557 91.694) (end 138.557 92.964) (width 0.2032) (layer "F.Cu") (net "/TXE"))
 (segment (start 138.811 93.218) (end 139.993999 93.218) (width 0.2032) (layer "F.Cu") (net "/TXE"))
 (via (at 143.581001 92.5034) (size 0.508) (drill 0.254) (layers "F.Cu" "B.Cu") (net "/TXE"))
 (segment (start 143.581001 92.5034) (end 143.255601 92.178) (width 0.3) (layer "B.Cu") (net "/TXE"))
 (segment (start 139.827 91.694) (end 138.557 91.694) (width 0.2032) (layer "B.Cu") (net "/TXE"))
 (segment (start 143.255601 92.178) (end 139.898001 92.178) (width 0.3) (layer "B.Cu") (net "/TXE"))
 (segment (start 138.557 89.154) (end 137.0402 90.6708) (width 0.3) (layer "F.Cu") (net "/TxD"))
 (segment (start 137.0402 95.338818) (end 138.007182 96.3058) (width 0.3) (layer "F.Cu") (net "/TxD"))
 (segment (start 138.007182 96.3058) (end 138.884818 96.3058) (width 0.3) (layer "F.Cu") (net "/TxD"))
 (segment (start 139.446 95.744618) (end 139.446 94.801) (width 0.3) (layer "F.Cu") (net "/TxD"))
 (segment (start 144.577501 91.243) (end 144.810001 91.4755) (width 0.2032) (layer "F.Cu") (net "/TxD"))
 (segment (start 138.884818 96.3058) (end 139.446 95.744618) (width 0.3) (layer "F.Cu") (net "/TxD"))
 (segment (start 137.0402 90.6708) (end 137.0402 95.338818) (width 0.3) (layer "F.Cu") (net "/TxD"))
 (segment (start 142.180001 89.638) (end 143.785001 91.243) (width 0.2032) (layer "F.Cu") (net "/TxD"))
 (segment (start 140.335 89.638) (end 140.311 89.638) (width 0.2032) (layer "F.Cu") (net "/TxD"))
 (segment (start 144.810001 95.352999) (end 144.556 95.607) (width 0.2032) (layer "F.Cu") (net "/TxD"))
 (segment (start 144.810001 91.4755) (end 144.810001 95.352999) (width 0.2032) (layer "F.Cu") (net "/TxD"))
 (segment (start 140.335 89.638) (end 142.180001 89.638) (width 0.2032) (layer "F.Cu") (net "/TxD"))
 (segment (start 143.785001 91.243) (end 144.577501 91.243) (width 0.2032) (layer "F.Cu") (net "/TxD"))
 (segment (start 140.311 89.638) (end 139.827 89.154) (width 0.2032) (layer "F.Cu") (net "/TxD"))
 (segment (start 144.556 95.607) (end 143.581001 95.607) (width 0.2032) (layer "F.Cu") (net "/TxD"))
 (segment (start 139.827 89.154) (end 138.557 89.154) (width 0.2032) (layer "B.Cu") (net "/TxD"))
 (segment (start 150.489801 96.959801) (end 150.495 96.965) (width 0.3) (layer "F.Cu") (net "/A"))
 (segment (start 152.090001 95.0355) (end 151.644501 94.59) (width 0.3) (layer "F.Cu") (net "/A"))
 (segment (start 151.644501 94.59) (end 150.489801 94.59) (width 0.3) (layer "F.Cu") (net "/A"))
 (segment (start 148.531001 94.337) (end 150.236801 94.337) (width 0.3) (layer "F.Cu") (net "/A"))
 (segment (start 150.489801 94.59) (end 150.489801 96.959801) (width 0.3) (layer "F.Cu") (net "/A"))
 (segment (start 150.236801 94.337) (end 150.489801 94.59) (width 0.3) (layer "F.Cu") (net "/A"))
 (segment (start 148.531001 93.067) (end 150.362801 93.067) (width 0.3) (layer "F.Cu") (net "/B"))
 (segment (start 150.489801 92.94) (end 151.645501 92.94) (width 0.3) (layer "F.Cu") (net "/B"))
 (segment (start 150.362801 93.067) (end 150.489801 92.94) (width 0.3) (layer "F.Cu") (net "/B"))
 (segment (start 150.495 90.741) (end 150.495 91.185) (width 0.3) (layer "F.Cu") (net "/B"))
 (segment (start 150.489801 92.94) (end 150.489801 90.746199) (width 0.3) (layer "F.Cu") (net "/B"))
 (segment (start 150.489801 90.746199) (end 150.495 90.741) (width 0.3) (layer "F.Cu") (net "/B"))
 (segment (start 151.645501 92.94) (end 152.090001 92.4955) (width 0.3) (layer "F.Cu") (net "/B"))
 (segment (start 147.975001 87.86) (end 147.975001 87.942) (width 0.3) (layer "F.Cu") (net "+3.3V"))
 (segment (start 145.928001 96.398001) (end 145.928001 94.869) (width 0.3) (layer "F.Cu") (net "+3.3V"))
 (segment (start 149.5494 94.9394) (end 150.006356 95.396356) (width 0.3) (layer "F.Cu") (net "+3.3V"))
 (segment (start 145.928001 94.869) (end 145.928001 89.989) (width 0.3) (layer "F.Cu") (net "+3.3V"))
 (segment (start 149.7176 96.551356) (end 149.7176 97.8376) (width 0.3) (layer "F.Cu") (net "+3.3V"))
 (segment (start 150.006356 96.2626) (end 149.7176 96.551356) (width 0.3) (layer "F.Cu") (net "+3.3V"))
 (segment (start 147.421 97.536) (end 147.414 97.543) (width 0.3) (layer "F.Cu") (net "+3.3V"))
 (segment (start 150.006356 95.396356) (end 150.006356 96.2626) (width 0.3) (layer "F.Cu") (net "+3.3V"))
 (segment (start 147.168 97.512) (end 147.199 97.543) (width 0.3) (layer "F.Cu") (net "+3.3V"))
 (segment (start 145.928001 94.869) (end 145.998401 94.9394) (width 0.3) (layer "F.Cu") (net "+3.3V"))
 (segment (start 145.998401 94.9394) (end 149.5494 94.9394) (width 0.3) (layer "F.Cu") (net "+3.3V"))
 (segment (start 147.975001 87.942) (end 147.168501 88.748501) (width 0.3) (layer "F.Cu") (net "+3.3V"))
 (segment (start 149.7176 97.8376) (end 150.495 98.615) (width 0.3) (layer "F.Cu") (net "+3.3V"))
 (segment (start 147.066 97.536) (end 145.928001 96.398001) (width 0.3) (layer "F.Cu") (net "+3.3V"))
 (segment (start 147.168501 88.748501) (end 145.928001 89.989) (width 0.3) (layer "F.Cu") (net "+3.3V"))
 (segment (start 146.055001 91.797) (end 148.531001 91.797) (width 0.3) (layer "F.Cu") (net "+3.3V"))
 (segment (start 135.922 88.678) (end 136.525 89.281) (width 0.3) (layer "F.Cu") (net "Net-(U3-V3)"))
 (segment (start 138.403354 93.445354) (end 138.446 93.488) (width 0.3) (layer "F.Cu") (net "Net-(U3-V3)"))
 (segment (start 135.375 88.678) (end 135.922 88.678) (width 0.3) (layer "F.Cu") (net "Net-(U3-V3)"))
 (segment (start 138.446 93.488) (end 138.446 94.42) (width 0.3) (layer "F.Cu") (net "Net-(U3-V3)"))
 (segment (start 138.319932 93.445354) (end 138.403354 93.445354) (width 0.3) (layer "F.Cu") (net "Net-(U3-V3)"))
 (via (at 138.319932 93.445354) (size 0.508) (drill 0.254) (layers "F.Cu" "B.Cu") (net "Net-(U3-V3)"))
 (via (at 136.525 89.281) (size 0.508) (drill 0.254) (layers "F.Cu" "B.Cu") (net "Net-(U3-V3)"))
 (segment (start 138.319932 93.445354) (end 136.525 91.650422) (width 0.3) (layer "B.Cu") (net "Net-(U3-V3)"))
 (segment (start 136.525 91.650422) (end 136.525 89.281) (width 0.3) (layer "B.Cu") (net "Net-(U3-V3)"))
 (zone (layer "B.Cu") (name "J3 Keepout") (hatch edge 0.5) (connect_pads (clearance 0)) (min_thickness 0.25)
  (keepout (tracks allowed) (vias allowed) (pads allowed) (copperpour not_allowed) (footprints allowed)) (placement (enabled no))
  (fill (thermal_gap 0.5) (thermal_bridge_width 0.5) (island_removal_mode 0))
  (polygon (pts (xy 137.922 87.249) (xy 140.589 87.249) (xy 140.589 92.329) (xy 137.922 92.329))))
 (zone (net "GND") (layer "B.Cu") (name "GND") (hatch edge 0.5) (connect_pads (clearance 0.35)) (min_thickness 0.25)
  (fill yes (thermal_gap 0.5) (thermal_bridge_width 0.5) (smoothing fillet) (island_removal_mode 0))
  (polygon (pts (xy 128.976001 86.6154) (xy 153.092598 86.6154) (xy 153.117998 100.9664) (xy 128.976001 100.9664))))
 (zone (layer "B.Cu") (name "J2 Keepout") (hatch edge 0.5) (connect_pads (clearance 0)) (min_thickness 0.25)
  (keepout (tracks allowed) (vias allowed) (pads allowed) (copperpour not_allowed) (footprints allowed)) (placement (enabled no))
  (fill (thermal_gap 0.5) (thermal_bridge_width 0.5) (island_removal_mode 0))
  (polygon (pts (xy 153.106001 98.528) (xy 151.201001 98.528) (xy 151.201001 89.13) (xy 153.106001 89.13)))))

